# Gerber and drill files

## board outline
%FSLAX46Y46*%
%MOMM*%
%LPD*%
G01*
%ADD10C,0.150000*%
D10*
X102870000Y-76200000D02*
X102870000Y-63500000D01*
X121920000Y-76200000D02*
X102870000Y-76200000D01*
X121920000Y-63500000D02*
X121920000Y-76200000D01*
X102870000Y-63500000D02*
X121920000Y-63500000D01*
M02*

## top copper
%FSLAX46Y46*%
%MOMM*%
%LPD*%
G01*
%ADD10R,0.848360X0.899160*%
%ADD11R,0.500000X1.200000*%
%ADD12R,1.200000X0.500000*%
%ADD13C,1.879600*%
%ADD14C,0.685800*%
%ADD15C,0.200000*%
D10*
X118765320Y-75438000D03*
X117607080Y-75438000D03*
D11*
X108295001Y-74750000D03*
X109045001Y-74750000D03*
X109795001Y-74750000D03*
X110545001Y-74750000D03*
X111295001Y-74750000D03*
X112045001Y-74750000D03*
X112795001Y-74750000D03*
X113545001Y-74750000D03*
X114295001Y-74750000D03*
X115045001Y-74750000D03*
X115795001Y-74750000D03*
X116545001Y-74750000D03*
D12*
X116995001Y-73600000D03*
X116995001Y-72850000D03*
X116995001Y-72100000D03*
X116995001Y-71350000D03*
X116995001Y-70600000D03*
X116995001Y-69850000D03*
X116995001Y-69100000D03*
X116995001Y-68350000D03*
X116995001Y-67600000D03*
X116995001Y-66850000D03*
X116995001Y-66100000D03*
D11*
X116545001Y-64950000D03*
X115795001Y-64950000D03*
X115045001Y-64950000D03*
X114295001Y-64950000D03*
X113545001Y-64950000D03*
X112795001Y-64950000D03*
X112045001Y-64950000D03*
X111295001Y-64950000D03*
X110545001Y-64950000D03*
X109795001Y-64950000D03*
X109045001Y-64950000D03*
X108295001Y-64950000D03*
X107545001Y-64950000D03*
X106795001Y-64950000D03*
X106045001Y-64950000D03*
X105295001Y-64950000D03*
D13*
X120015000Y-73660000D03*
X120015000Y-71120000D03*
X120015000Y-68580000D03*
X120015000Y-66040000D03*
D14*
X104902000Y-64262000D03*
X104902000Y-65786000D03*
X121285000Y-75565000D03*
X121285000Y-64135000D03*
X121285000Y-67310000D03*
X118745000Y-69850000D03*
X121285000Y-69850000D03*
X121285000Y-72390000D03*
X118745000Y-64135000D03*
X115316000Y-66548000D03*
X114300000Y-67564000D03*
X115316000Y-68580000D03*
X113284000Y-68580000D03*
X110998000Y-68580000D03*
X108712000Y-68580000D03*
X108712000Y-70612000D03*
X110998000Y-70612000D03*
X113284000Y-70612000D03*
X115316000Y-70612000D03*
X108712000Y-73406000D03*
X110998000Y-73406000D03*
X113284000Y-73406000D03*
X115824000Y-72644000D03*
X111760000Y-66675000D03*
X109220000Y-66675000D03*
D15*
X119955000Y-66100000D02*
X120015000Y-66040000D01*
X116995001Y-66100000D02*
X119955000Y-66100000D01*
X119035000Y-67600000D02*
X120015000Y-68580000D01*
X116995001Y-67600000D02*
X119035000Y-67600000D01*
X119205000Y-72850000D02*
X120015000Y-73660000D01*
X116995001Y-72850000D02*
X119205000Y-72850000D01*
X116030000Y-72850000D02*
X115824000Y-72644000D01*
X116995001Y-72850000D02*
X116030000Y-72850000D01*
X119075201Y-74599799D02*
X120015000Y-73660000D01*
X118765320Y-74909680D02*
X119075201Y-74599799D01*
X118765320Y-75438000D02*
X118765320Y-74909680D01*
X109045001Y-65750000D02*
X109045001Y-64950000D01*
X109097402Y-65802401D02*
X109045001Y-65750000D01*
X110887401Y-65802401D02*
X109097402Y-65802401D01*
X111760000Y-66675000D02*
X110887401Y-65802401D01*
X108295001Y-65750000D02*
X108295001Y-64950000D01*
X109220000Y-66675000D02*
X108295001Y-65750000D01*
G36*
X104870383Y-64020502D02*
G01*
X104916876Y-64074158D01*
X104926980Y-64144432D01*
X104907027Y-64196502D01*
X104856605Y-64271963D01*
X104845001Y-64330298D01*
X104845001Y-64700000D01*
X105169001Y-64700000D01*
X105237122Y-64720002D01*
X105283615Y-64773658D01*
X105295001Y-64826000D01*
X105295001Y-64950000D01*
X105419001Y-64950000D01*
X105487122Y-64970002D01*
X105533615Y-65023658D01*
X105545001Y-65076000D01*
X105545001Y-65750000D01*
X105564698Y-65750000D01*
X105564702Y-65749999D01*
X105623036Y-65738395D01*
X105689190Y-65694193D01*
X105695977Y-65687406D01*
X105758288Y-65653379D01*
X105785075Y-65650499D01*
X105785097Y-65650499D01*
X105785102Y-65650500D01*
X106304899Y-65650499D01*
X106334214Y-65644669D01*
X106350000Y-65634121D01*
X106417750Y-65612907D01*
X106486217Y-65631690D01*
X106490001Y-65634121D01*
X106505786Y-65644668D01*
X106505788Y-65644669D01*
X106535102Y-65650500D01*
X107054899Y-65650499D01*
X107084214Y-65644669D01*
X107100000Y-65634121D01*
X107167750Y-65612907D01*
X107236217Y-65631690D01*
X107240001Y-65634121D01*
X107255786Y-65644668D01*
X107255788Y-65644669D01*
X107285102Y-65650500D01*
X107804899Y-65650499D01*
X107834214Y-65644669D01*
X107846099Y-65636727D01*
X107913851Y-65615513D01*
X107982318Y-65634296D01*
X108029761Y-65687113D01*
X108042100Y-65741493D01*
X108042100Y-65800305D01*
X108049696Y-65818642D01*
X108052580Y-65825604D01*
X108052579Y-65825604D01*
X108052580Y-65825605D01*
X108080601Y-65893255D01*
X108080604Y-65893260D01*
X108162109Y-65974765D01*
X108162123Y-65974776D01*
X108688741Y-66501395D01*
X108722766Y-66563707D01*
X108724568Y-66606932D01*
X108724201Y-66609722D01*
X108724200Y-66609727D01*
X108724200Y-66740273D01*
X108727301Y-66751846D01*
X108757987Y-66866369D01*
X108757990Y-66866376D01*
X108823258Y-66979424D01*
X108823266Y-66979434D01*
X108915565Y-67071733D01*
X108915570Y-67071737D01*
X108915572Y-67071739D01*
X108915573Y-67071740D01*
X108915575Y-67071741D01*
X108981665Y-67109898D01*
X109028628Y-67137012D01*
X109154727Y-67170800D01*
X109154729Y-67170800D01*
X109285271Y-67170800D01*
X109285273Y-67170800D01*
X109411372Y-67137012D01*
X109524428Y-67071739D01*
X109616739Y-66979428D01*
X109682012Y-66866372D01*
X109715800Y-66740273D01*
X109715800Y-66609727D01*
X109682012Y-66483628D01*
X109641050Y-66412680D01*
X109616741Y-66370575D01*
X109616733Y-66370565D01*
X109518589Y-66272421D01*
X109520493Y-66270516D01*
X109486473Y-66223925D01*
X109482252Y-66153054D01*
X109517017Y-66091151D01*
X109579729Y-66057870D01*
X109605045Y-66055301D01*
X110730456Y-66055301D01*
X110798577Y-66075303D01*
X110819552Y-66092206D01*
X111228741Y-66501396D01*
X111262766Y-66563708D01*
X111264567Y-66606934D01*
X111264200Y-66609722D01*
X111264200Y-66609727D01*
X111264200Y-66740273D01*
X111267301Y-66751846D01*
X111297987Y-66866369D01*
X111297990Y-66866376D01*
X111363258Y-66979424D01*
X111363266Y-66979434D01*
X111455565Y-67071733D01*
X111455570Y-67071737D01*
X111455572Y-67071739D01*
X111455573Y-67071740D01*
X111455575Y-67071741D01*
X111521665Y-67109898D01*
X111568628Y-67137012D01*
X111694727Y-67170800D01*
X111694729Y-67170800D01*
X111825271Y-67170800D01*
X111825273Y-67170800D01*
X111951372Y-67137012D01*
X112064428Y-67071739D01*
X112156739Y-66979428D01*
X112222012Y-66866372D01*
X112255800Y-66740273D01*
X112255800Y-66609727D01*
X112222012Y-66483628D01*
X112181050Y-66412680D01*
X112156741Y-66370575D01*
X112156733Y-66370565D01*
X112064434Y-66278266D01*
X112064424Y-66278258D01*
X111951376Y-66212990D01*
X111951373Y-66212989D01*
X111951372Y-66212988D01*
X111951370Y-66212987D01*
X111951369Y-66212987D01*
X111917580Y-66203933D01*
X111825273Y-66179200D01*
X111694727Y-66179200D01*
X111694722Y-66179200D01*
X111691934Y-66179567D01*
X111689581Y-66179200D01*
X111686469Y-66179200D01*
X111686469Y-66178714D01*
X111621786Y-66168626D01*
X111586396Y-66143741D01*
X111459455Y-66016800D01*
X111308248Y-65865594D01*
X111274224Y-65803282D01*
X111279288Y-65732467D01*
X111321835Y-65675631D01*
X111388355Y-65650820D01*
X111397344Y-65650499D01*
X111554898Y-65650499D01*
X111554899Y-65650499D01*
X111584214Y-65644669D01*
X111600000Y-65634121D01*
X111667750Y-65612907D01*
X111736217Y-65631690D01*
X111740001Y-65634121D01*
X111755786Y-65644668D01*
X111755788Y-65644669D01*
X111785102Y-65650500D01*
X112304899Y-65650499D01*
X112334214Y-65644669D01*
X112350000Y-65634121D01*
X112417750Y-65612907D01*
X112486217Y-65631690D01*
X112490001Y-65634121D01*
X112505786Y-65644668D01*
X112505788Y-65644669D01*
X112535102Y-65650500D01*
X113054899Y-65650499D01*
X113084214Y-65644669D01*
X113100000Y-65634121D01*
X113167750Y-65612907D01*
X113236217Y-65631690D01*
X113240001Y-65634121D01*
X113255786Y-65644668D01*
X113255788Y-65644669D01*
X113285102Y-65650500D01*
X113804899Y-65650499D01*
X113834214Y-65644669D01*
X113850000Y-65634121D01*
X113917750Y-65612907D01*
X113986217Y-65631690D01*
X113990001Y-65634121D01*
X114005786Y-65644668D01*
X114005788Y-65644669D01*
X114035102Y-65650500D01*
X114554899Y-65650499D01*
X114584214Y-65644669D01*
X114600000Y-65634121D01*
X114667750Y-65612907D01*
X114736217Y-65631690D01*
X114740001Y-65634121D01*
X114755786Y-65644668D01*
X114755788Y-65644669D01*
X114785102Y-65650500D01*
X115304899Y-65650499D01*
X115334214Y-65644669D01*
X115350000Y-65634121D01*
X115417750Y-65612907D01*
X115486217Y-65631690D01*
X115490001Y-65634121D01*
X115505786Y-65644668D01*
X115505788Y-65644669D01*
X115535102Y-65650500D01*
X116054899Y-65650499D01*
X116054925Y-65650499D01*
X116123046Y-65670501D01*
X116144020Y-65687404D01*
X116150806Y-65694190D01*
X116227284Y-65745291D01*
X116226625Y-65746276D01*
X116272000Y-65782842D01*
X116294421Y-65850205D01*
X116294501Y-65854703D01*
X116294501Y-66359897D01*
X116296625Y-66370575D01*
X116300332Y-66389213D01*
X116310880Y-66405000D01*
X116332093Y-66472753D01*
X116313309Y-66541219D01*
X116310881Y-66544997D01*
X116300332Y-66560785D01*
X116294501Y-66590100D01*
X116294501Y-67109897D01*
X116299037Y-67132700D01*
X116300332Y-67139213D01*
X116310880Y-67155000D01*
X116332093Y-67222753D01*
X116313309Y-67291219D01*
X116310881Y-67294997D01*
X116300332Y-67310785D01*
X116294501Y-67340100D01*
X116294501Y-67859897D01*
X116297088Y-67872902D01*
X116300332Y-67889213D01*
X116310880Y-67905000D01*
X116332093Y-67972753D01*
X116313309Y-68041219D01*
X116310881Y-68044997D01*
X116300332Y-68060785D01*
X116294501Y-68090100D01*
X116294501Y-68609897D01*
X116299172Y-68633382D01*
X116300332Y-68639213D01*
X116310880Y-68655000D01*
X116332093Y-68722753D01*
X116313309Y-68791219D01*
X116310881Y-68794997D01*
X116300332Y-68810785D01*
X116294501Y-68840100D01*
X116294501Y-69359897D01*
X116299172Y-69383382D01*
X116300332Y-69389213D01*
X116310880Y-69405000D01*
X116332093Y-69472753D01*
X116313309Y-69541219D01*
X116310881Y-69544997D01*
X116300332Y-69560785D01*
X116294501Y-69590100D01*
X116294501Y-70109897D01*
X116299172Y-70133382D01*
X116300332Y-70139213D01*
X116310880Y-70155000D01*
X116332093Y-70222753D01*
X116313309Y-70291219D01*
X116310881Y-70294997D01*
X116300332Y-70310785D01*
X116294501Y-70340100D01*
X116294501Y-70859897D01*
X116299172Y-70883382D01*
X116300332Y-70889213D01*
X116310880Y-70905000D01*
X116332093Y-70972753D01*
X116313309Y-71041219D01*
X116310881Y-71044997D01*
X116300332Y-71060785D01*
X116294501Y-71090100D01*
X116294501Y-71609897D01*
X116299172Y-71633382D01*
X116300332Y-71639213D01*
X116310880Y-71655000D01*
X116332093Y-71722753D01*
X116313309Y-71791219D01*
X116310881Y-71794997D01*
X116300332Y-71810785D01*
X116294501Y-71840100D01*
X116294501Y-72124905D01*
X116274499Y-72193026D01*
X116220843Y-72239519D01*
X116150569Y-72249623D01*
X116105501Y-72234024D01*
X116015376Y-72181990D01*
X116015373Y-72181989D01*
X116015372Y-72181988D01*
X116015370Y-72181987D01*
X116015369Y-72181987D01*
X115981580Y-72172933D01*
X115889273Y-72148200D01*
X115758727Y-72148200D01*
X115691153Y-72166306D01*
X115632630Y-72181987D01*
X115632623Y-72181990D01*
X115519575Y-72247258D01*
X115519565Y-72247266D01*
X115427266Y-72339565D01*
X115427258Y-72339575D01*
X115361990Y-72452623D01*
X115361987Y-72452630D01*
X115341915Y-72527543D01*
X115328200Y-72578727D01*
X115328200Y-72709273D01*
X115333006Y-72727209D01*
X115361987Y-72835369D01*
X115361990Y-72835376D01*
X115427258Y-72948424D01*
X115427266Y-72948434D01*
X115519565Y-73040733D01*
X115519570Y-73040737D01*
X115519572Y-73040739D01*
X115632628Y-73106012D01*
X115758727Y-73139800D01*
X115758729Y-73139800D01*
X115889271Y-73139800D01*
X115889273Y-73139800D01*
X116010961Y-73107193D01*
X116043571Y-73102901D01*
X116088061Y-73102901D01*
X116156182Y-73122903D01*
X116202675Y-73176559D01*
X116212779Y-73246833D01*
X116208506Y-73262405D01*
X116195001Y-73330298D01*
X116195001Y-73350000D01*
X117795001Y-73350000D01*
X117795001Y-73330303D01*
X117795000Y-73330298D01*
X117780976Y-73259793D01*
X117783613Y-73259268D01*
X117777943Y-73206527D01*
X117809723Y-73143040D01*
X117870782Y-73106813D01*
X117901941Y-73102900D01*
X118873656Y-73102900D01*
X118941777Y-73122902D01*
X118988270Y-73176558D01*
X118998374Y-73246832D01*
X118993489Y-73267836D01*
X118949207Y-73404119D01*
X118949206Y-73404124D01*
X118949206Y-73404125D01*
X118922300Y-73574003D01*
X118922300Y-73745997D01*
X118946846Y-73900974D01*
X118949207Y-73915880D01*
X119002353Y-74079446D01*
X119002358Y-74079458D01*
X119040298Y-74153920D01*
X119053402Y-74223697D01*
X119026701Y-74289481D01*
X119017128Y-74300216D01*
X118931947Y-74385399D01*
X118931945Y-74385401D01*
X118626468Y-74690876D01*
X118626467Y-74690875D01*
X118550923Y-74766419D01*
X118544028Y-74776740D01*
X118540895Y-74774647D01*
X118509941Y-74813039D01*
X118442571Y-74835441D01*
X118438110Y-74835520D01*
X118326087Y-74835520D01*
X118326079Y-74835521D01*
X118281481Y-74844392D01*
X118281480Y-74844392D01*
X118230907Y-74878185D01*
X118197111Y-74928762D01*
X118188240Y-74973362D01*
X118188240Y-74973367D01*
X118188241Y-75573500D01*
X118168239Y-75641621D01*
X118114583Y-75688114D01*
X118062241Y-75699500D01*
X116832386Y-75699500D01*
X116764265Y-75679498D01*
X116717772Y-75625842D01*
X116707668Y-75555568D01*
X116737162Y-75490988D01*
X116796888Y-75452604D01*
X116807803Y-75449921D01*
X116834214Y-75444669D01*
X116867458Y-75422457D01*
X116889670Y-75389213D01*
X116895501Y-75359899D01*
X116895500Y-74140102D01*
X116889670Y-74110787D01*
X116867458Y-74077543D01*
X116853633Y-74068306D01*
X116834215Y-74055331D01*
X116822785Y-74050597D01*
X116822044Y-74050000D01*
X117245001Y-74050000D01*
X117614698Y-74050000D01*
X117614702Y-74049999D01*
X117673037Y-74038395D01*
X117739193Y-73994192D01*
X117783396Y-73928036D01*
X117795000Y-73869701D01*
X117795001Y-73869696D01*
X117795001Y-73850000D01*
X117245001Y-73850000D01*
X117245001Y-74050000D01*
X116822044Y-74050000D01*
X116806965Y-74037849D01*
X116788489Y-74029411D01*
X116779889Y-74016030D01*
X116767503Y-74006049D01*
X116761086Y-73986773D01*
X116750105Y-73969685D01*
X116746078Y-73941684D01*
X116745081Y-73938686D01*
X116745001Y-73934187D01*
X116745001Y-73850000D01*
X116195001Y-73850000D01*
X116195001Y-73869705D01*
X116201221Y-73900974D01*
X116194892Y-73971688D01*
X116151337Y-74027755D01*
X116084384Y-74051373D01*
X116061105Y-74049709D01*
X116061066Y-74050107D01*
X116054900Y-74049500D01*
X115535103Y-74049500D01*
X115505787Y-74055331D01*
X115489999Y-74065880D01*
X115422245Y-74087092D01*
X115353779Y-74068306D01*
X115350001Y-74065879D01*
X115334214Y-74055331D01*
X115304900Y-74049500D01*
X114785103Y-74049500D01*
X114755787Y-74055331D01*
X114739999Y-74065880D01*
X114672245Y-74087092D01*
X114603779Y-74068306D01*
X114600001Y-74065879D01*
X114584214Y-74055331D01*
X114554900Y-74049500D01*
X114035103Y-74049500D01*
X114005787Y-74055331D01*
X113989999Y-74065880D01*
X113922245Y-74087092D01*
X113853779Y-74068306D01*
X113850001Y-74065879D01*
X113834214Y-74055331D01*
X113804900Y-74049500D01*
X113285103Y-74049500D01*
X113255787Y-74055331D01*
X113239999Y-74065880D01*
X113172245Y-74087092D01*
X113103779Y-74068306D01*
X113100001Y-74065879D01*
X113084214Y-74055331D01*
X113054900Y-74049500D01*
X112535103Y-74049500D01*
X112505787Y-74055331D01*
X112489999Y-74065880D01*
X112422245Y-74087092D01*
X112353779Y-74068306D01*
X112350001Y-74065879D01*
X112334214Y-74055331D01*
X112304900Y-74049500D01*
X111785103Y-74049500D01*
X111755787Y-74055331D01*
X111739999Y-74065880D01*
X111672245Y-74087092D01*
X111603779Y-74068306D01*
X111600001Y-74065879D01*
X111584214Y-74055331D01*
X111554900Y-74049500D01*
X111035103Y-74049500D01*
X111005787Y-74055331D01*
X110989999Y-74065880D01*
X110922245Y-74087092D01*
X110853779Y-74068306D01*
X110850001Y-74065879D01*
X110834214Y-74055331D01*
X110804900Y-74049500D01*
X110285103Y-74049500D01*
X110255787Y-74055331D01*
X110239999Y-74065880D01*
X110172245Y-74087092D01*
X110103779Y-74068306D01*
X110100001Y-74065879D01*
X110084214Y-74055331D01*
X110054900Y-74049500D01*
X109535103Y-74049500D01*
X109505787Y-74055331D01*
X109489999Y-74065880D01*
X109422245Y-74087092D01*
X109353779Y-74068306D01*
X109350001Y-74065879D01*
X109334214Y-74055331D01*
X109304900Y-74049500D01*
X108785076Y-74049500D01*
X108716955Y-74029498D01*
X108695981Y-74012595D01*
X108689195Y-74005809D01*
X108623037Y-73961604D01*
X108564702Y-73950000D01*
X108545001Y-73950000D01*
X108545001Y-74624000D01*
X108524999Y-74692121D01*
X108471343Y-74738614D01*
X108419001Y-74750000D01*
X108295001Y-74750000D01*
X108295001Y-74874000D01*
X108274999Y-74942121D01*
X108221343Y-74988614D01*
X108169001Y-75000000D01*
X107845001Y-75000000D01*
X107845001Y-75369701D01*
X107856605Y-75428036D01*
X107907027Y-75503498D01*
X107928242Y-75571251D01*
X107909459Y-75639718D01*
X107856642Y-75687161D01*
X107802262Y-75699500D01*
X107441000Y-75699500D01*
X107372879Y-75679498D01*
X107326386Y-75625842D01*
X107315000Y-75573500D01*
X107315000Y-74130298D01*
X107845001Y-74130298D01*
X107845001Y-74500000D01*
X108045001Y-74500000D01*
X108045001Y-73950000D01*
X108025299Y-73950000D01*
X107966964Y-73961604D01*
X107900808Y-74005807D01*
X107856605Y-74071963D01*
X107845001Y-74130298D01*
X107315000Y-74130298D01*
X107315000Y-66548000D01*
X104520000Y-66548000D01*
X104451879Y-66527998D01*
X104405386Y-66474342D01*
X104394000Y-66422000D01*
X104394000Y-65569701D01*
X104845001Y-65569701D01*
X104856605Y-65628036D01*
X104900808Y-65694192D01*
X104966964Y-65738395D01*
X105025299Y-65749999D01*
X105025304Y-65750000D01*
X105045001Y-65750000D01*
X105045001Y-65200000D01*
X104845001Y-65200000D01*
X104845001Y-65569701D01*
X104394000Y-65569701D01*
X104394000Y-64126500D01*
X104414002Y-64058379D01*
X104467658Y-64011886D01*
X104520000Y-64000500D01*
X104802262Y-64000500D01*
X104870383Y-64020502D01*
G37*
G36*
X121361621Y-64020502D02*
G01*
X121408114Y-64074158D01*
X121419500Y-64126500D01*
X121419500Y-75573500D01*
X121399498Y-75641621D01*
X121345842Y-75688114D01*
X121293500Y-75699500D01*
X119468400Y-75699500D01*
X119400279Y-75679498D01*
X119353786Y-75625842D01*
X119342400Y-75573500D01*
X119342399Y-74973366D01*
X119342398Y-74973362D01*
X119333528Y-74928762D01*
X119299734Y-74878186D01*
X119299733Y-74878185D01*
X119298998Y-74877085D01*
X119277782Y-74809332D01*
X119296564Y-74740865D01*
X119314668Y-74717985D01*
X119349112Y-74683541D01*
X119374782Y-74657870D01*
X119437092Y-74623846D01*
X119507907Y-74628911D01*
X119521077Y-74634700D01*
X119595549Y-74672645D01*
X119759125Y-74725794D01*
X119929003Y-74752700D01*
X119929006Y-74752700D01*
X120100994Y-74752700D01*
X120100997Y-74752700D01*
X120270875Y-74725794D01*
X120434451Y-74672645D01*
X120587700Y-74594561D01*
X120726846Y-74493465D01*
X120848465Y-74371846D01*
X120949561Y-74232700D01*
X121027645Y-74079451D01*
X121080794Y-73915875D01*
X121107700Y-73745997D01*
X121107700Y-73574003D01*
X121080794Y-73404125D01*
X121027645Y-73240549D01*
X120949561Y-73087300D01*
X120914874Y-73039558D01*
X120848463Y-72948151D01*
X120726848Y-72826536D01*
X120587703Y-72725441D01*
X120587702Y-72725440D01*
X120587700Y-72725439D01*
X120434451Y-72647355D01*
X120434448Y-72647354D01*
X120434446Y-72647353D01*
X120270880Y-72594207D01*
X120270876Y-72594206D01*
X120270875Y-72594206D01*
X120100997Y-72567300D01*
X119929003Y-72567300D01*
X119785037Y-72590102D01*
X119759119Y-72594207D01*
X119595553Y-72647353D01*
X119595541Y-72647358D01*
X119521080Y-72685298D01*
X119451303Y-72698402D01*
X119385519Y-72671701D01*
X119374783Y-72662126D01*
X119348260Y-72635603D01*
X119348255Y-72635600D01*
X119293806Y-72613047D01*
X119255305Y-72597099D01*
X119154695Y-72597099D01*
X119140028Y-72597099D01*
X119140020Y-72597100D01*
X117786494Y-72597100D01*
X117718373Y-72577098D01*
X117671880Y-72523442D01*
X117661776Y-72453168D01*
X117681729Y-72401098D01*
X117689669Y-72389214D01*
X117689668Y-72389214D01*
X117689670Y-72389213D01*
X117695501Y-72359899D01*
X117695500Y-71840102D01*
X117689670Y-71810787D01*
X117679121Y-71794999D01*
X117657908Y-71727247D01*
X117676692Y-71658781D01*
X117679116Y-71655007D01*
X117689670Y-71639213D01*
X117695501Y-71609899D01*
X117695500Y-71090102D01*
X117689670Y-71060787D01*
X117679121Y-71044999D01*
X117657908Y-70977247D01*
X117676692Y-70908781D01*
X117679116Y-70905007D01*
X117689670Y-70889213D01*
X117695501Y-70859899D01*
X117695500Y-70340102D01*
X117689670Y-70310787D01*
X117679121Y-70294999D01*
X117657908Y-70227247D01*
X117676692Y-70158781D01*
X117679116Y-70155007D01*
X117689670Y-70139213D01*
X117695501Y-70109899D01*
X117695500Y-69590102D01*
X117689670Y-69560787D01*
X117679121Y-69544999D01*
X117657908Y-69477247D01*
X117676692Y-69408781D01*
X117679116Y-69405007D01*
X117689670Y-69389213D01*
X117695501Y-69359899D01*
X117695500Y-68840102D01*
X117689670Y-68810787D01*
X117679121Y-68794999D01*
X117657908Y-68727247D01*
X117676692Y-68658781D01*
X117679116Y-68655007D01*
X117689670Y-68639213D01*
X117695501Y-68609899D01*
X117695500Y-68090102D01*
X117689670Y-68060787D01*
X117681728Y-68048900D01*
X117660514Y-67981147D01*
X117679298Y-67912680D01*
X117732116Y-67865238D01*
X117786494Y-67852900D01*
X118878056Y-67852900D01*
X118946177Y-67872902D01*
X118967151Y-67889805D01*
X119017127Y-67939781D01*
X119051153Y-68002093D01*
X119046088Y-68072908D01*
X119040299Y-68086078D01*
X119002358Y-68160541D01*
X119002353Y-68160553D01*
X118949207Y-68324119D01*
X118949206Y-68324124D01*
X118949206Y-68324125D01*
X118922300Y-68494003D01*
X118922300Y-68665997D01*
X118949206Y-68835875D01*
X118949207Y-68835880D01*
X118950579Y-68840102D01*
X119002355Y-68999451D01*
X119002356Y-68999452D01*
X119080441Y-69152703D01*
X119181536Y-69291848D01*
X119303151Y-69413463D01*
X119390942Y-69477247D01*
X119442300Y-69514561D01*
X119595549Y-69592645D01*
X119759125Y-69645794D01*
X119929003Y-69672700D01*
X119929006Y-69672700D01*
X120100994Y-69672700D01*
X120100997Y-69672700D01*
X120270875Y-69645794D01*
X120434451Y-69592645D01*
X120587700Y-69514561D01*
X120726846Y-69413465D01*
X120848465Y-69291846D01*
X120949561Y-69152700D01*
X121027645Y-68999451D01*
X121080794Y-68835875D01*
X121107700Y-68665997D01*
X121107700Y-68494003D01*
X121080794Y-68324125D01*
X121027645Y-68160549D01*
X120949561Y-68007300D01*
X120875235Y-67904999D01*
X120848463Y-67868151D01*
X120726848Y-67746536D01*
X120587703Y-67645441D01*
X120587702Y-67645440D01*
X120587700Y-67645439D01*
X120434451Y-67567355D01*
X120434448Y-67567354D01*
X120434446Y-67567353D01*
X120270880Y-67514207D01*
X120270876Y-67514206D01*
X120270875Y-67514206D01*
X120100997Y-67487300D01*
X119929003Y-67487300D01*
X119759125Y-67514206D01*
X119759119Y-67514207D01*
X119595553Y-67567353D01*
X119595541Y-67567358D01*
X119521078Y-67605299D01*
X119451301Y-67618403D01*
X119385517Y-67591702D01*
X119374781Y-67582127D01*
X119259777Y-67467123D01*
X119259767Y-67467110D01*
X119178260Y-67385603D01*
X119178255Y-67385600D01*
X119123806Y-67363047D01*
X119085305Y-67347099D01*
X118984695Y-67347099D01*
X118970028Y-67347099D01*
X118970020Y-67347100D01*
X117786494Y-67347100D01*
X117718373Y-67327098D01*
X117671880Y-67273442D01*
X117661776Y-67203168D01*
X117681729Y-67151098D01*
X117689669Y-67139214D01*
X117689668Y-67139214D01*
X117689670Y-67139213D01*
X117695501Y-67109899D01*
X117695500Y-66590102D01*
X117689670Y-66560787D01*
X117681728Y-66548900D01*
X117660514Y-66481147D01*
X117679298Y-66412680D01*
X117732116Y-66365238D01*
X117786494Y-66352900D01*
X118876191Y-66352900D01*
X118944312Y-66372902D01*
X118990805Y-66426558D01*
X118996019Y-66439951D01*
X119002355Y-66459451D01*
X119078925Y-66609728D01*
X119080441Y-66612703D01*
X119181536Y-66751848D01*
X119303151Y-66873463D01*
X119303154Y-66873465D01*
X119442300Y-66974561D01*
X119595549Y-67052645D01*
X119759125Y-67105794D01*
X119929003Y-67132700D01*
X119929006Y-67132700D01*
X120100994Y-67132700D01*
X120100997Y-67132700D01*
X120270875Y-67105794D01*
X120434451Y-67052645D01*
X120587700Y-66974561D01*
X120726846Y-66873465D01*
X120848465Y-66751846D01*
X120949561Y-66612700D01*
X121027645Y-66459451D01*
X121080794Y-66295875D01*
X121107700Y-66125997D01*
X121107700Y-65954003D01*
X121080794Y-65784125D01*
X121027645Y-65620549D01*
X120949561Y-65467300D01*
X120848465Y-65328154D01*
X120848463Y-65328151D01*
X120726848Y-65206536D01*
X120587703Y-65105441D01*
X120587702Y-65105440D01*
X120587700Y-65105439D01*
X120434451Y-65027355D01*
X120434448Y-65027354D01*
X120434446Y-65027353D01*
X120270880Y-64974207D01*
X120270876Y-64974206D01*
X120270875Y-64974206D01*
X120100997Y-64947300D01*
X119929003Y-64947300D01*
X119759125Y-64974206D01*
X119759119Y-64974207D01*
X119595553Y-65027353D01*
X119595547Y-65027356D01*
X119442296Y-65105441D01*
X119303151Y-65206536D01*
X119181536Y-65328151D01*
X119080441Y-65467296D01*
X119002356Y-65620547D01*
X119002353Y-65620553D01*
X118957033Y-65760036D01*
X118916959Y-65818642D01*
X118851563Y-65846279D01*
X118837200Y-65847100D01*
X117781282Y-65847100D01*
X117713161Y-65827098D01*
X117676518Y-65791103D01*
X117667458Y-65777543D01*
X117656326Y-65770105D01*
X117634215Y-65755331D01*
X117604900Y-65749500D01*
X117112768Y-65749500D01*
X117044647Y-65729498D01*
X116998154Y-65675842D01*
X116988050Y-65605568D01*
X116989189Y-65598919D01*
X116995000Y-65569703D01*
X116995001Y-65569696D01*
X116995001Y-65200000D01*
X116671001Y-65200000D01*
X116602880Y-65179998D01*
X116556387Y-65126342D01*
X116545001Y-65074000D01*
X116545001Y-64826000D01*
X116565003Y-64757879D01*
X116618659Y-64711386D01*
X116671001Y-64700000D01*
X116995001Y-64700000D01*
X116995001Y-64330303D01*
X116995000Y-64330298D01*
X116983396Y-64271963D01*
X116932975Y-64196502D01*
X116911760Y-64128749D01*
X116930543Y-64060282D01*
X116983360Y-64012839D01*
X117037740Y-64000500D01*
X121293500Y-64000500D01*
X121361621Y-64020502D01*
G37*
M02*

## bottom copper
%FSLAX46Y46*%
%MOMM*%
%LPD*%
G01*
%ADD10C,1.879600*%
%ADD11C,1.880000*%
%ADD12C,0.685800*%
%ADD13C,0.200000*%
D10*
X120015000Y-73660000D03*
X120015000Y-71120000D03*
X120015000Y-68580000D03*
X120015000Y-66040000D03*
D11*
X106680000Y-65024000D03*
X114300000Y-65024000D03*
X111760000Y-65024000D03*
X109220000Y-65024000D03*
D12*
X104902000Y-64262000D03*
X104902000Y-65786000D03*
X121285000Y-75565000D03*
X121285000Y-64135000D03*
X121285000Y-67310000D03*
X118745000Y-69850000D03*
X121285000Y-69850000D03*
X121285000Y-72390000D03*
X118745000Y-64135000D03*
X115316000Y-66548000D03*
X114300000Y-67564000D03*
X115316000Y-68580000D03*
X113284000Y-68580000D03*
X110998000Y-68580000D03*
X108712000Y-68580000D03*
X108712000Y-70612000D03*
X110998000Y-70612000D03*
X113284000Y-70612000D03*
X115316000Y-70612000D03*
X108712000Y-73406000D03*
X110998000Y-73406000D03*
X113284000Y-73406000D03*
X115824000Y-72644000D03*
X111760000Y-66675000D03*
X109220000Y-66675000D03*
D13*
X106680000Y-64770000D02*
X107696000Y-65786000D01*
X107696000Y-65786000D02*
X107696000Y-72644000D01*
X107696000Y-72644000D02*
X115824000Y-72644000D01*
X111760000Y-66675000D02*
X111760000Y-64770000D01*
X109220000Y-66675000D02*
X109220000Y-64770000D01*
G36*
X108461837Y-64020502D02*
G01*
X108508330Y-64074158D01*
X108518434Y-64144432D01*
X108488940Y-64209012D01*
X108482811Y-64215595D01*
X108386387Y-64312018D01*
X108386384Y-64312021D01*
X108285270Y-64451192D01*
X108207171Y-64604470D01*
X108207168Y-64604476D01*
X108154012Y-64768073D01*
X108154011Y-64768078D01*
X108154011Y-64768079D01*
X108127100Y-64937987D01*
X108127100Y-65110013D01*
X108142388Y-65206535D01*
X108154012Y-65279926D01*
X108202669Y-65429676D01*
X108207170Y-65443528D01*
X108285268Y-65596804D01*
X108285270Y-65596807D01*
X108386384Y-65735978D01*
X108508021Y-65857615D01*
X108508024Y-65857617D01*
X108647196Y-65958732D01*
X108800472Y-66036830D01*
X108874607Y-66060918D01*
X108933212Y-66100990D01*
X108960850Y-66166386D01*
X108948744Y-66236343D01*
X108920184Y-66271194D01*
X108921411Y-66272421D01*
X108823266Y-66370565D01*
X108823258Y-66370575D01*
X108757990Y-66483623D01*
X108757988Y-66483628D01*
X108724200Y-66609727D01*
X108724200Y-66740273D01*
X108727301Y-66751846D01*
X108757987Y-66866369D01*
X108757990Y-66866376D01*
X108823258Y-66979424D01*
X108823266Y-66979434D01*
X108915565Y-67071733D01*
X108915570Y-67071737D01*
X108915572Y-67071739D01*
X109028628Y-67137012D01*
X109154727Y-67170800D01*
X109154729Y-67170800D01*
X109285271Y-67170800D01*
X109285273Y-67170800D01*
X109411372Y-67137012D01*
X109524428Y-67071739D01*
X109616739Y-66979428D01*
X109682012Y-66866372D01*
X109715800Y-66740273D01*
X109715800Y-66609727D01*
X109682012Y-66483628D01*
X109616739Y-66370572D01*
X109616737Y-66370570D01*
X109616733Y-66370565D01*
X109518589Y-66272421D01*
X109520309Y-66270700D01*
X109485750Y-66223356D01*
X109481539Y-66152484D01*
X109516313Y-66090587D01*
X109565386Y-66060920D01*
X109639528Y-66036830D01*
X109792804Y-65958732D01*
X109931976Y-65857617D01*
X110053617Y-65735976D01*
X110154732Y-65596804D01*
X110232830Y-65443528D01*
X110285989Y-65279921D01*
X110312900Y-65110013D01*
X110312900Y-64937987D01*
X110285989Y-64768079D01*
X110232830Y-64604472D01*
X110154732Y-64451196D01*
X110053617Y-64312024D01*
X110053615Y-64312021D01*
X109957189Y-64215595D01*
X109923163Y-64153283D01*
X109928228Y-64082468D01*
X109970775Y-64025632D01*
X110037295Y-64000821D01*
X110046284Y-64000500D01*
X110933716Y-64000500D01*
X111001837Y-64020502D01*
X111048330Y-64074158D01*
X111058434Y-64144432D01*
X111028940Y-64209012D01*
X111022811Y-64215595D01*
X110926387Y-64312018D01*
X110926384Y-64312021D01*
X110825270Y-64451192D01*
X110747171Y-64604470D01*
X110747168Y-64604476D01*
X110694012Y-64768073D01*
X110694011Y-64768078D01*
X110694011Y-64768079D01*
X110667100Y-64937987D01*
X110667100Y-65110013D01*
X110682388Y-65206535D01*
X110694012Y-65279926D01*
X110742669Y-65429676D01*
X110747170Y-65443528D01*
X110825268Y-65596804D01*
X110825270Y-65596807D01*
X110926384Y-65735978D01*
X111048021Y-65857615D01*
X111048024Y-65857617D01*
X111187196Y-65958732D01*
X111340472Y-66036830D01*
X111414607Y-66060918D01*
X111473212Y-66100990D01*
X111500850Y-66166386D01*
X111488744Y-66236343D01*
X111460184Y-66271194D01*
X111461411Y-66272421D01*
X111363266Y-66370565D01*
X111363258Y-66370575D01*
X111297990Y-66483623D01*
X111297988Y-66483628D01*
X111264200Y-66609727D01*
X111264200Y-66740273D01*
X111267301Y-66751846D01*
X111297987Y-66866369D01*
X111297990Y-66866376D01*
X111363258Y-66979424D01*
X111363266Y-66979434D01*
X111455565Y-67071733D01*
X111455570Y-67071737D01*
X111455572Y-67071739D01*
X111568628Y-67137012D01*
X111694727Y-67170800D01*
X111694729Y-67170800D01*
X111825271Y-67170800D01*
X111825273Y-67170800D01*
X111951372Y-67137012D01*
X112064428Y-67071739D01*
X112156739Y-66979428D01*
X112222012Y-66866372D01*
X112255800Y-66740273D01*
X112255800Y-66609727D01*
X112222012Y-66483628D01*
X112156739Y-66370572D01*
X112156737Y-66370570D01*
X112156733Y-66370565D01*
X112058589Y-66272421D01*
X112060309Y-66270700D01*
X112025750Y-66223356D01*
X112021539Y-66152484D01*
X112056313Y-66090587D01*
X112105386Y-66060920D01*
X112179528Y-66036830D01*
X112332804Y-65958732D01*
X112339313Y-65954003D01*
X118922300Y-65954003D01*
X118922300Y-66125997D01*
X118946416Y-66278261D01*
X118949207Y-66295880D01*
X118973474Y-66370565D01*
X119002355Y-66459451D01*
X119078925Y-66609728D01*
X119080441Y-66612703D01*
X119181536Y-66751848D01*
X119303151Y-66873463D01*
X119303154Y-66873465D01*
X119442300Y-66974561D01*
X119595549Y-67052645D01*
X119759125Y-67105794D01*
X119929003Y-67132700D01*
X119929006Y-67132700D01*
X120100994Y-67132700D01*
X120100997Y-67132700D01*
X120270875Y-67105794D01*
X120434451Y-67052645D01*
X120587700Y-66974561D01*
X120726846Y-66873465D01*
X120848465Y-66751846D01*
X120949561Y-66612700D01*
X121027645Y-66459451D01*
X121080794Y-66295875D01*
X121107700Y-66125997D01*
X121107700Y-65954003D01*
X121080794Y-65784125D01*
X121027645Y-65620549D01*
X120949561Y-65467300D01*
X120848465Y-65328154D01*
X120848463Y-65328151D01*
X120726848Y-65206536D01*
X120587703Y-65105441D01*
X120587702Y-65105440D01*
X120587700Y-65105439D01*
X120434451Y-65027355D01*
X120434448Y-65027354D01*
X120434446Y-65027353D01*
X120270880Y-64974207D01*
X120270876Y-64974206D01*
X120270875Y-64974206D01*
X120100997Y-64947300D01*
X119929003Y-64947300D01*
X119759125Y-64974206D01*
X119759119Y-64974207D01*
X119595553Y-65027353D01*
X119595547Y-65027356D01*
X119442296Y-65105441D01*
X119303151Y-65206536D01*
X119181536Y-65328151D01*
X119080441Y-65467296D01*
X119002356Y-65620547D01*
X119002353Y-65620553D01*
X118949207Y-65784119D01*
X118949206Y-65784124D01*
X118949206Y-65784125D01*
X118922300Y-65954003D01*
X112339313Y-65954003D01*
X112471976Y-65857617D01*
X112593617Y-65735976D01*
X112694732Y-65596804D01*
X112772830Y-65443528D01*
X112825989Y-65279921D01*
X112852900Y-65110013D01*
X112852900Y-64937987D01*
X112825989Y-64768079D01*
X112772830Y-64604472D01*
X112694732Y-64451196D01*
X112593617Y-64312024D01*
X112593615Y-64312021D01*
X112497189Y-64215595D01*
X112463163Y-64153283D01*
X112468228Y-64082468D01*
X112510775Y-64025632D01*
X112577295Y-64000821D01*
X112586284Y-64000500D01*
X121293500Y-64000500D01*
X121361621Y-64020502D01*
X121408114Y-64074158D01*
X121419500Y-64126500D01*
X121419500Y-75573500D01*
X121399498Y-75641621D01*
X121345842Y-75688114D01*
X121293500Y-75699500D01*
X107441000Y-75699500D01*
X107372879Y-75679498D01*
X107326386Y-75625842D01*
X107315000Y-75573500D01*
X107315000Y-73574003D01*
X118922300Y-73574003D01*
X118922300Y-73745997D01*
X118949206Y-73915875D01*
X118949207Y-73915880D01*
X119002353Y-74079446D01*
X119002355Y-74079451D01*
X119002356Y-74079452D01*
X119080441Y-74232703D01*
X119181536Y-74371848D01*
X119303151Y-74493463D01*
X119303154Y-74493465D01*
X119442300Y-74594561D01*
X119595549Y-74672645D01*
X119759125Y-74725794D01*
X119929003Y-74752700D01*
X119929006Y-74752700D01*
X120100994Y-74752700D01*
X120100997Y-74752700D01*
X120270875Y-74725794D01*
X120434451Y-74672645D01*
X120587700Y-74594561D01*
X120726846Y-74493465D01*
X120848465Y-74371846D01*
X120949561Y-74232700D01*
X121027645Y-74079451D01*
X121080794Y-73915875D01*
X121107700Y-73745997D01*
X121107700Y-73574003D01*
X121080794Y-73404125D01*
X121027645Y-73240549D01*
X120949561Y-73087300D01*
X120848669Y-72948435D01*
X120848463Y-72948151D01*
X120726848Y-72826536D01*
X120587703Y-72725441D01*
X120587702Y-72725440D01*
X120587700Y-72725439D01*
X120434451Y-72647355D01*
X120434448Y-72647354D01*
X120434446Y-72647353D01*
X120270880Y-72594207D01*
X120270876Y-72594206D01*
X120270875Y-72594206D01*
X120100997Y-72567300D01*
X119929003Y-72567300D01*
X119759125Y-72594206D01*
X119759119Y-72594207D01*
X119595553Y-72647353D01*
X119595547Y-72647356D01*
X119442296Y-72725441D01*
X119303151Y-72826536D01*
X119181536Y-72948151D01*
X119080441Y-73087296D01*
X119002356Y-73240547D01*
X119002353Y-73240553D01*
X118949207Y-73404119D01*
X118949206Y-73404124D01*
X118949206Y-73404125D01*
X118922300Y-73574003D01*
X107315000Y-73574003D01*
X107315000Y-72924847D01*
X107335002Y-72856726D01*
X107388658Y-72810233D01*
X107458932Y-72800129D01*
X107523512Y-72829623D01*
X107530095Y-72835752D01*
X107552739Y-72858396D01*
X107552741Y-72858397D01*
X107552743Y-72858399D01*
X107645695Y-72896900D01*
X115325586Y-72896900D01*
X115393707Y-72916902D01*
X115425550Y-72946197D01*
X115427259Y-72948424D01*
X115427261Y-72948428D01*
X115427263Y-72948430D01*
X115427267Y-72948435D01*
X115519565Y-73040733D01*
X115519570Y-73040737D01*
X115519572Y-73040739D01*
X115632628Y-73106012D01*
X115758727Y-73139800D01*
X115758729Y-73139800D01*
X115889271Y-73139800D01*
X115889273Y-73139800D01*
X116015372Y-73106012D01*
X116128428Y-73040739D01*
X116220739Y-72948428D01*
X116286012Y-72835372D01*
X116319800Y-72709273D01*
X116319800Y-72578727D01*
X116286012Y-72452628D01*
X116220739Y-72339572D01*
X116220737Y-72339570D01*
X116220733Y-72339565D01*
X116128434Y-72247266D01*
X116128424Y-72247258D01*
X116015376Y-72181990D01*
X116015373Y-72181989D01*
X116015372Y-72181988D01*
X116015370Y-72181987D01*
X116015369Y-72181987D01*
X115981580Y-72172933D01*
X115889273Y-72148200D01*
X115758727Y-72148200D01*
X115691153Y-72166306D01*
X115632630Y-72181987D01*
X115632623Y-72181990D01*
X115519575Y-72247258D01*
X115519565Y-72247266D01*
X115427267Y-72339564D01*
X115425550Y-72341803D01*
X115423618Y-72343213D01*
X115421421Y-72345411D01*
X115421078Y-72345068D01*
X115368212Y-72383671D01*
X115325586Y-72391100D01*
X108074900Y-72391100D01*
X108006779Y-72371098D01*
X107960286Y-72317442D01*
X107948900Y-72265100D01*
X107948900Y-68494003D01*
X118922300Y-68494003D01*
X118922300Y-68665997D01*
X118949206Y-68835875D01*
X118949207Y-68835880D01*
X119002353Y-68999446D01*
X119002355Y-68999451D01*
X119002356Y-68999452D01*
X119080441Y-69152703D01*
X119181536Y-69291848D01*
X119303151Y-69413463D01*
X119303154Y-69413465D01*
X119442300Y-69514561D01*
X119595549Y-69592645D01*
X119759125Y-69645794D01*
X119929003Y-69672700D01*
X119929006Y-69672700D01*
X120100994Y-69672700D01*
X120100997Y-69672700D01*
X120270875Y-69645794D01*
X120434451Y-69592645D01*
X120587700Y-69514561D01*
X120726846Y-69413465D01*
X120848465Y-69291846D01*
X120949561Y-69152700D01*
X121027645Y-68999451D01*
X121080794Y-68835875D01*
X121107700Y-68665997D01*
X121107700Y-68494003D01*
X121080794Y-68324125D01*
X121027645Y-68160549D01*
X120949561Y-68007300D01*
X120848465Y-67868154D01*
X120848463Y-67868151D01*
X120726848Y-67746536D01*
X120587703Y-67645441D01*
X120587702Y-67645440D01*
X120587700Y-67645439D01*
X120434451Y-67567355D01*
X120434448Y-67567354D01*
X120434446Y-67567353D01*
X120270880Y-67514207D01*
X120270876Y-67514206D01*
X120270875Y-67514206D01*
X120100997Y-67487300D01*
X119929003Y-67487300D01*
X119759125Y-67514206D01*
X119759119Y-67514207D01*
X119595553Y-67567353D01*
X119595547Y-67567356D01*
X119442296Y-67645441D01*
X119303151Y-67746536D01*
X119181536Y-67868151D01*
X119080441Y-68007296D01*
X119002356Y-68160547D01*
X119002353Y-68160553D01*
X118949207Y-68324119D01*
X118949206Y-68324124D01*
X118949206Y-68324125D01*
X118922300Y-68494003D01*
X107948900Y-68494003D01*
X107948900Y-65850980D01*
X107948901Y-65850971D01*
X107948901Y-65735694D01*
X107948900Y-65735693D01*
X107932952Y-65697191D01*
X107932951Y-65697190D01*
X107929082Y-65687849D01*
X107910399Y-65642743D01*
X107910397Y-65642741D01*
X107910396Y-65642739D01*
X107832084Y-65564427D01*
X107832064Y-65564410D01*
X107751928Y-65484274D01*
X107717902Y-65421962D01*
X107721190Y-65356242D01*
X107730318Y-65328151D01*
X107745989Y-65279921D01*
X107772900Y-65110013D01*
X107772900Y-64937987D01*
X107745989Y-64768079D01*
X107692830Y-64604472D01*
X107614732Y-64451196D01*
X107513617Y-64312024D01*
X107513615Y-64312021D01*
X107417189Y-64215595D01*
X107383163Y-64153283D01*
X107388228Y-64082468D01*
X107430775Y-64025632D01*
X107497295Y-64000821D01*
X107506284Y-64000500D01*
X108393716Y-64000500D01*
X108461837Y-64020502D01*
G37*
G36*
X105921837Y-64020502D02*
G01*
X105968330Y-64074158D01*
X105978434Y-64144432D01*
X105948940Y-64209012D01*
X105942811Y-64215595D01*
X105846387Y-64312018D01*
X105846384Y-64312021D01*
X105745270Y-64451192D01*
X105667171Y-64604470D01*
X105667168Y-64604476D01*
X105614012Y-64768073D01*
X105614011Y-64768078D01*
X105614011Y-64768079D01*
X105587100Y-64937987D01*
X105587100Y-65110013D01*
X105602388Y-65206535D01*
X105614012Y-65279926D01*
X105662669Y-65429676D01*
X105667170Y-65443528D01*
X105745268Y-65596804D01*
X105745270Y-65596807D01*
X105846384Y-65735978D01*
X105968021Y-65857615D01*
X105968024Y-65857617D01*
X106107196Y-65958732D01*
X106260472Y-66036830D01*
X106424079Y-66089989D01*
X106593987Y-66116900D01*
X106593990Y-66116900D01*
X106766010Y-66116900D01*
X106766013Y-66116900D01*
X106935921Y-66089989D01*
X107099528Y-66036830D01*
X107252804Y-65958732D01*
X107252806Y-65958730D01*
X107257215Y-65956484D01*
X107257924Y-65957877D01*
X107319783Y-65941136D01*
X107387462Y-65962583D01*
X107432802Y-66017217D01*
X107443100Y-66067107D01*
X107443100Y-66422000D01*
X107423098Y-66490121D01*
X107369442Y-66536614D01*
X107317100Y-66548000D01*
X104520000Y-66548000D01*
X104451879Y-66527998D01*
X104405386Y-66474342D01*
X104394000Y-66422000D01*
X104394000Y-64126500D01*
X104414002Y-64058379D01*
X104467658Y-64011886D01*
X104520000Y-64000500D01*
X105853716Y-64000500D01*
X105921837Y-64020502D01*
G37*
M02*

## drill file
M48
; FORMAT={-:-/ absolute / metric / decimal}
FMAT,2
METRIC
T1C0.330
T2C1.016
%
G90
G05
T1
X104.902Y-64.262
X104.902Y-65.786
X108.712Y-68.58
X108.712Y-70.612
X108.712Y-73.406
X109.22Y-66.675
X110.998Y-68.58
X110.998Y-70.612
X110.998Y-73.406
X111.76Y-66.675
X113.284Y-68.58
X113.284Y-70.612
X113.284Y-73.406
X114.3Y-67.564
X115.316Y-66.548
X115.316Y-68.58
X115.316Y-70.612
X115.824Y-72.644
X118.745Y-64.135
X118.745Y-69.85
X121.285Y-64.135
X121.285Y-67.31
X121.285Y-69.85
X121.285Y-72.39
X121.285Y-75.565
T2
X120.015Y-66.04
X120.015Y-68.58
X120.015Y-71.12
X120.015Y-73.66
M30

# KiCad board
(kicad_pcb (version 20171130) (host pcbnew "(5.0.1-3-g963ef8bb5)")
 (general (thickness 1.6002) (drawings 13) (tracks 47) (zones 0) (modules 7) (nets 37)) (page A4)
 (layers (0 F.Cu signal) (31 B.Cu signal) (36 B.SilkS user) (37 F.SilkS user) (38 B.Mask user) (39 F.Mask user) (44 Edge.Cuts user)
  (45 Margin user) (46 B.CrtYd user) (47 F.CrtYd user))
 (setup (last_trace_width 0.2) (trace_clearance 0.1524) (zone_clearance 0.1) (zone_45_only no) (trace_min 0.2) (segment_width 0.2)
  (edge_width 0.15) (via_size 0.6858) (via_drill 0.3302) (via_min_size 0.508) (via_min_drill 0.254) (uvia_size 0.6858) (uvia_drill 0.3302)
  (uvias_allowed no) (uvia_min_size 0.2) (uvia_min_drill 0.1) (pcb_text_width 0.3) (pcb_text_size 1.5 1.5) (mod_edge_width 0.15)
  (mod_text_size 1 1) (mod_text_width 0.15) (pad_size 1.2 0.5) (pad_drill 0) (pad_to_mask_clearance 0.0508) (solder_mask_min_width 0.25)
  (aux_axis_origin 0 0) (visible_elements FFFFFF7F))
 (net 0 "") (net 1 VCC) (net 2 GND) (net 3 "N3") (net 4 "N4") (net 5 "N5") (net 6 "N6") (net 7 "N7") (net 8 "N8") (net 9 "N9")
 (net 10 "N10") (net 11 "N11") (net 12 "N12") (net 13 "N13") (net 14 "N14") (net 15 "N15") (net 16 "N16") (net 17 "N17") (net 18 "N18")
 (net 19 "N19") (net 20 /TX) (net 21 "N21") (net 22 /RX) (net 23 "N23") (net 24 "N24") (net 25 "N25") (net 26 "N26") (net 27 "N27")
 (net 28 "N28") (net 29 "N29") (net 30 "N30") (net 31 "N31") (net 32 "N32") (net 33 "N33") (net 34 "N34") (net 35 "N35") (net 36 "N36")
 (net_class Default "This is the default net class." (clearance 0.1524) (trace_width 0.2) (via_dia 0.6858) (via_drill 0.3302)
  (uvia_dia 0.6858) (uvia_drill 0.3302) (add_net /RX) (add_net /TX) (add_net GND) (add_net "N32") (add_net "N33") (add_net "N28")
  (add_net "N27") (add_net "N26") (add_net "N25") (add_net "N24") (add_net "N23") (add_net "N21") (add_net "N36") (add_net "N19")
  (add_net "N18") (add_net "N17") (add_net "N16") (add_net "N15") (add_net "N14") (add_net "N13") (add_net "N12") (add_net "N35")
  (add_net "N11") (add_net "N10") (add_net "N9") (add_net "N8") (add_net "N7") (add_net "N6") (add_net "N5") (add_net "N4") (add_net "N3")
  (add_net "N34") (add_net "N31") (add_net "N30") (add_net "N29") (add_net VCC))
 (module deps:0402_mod (layer F.Cu) (at 118.1862 75.438 180)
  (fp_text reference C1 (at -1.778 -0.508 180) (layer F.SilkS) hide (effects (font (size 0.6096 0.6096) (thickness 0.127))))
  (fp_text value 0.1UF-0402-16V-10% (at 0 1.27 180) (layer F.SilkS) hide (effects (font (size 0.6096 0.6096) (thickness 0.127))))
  (pad 1 smd rect (at -0.57912 0 180) (size 0.84836 0.89916) (layers F.Cu F.Paste F.Mask) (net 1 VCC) (solder_mask_margin 0.1016))
  (pad 2 smd rect (at 0.57912 0 180) (size 0.84836 0.89916) (layers F.Cu F.Paste F.Mask) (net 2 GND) (solder_mask_margin 0.1016)))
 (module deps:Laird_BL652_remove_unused (layer F.Cu) (at 111.145001 69.85) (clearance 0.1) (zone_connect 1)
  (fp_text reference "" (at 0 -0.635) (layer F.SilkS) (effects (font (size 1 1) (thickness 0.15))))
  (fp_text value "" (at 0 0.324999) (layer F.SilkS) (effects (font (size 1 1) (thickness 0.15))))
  (pad 39 smd rect (at -2.85 4.9 90) (size 1.2 0.5) (layers F.Cu F.Paste F.Mask) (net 2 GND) (zone_connect 1))
  (pad 38 smd rect (at -2.1 4.9 90) (size 1.2 0.5) (layers F.Cu F.Paste F.Mask) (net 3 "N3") (zone_connect 1))
  (pad 37 smd rect (at -1.35 4.9 90) (size 1.2 0.5) (layers F.Cu F.Paste F.Mask) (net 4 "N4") (zone_connect 1))
  (pad 36 smd rect (at -0.6 4.9 90) (size 1.2 0.5) (layers F.Cu F.Paste F.Mask) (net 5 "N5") (zone_connect 1))
  (pad 35 smd rect (at 0.15 4.9 90) (size 1.2 0.5) (layers F.Cu F.Paste F.Mask) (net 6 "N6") (zone_connect 1))
  (pad 34 smd rect (at 0.9 4.9 90) (size 1.2 0.5) (layers F.Cu F.Paste F.Mask) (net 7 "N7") (zone_connect 1))
  (pad 33 smd rect (at 1.65 4.9 90) (size 1.2 0.5) (layers F.Cu F.Paste F.Mask) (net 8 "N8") (zone_connect 1))
  (pad 32 smd rect (at 2.4 4.9 90) (size 1.2 0.5) (layers F.Cu F.Paste F.Mask) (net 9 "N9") (zone_connect 1))
  (pad 31 smd rect (at 3.15 4.9 90) (size 1.2 0.5) (layers F.Cu F.Paste F.Mask) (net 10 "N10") (zone_connect 1))
  (pad 30 smd rect (at 3.9 4.9 90) (size 1.2 0.5) (layers F.Cu F.Paste F.Mask) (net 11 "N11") (zone_connect 1))
  (pad 29 smd rect (at 4.65 4.9 90) (size 1.2 0.5) (layers F.Cu F.Paste F.Mask) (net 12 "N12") (zone_connect 1))
  (pad 28 smd rect (at 5.4 4.9 90) (size 1.2 0.5) (layers F.Cu F.Paste F.Mask) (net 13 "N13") (zone_connect 1))
  (pad 27 smd rect (at 5.85 3.75) (size 1.2 0.5) (layers F.Cu F.Paste F.Mask) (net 2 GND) (zone_connect 1))
  (pad 26 smd rect (at 5.85 3) (size 1.2 0.5) (layers F.Cu F.Paste F.Mask) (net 1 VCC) (zone_connect 1))
  (pad 25 smd rect (at 5.85 2.25) (size 1.2 0.5) (layers F.Cu F.Paste F.Mask) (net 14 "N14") (zone_connect 1))
  (pad 24 smd rect (at 5.85 1.5) (size 1.2 0.5) (layers F.Cu F.Paste F.Mask) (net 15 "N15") (zone_connect 1))
  (pad 23 smd rect (at 5.85 0.75) (size 1.2 0.5) (layers F.Cu F.Paste F.Mask) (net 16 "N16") (zone_connect 1))
  (pad 22 smd rect (at 5.85 0) (size 1.2 0.5) (layers F.Cu F.Paste F.Mask) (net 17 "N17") (zone_connect 1))
  (pad 21 smd rect (at 5.85 -0.75) (size 1.2 0.5) (layers F.Cu F.Paste F.Mask) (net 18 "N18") (zone_connect 1))
  (pad 20 smd rect (at 5.85 -1.5) (size 1.2 0.5) (layers F.Cu F.Paste F.Mask) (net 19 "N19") (zone_connect 1))
  (pad 19 smd rect (at 5.85 -2.25) (size 1.2 0.5) (layers F.Cu F.Paste F.Mask) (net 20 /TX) (zone_connect 1))
  (pad 18 smd rect (at 5.85 -3) (size 1.2 0.5) (layers F.Cu F.Paste F.Mask) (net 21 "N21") (zone_connect 1))
  (pad 17 smd rect (at 5.85 -3.75) (size 1.2 0.5) (layers F.Cu F.Paste F.Mask) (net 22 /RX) (zone_connect 1))
  (pad 16 smd rect (at 5.4 -4.9 90) (size 1.2 0.5) (layers F.Cu F.Paste F.Mask) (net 2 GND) (zone_connect 1))
  (pad 15 smd rect (at 4.65 -4.9 90) (size 1.2 0.5) (layers F.Cu F.Paste F.Mask) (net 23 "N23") (zone_connect 1))
  (pad 14 smd rect (at 3.9 -4.9 90) (size 1.2 0.5) (layers F.Cu F.Paste F.Mask) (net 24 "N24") (zone_connect 1))
  (pad 13 smd rect (at 3.15 -4.9 90) (size 1.2 0.5) (layers F.Cu F.Paste F.Mask) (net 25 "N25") (zone_connect 1))
  (pad 12 smd rect (at 2.4 -4.9 90) (size 1.2 0.5) (layers F.Cu F.Paste F.Mask) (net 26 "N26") (zone_connect 1))
  (pad 11 smd rect (at 1.65 -4.9 90) (size 1.2 0.5) (layers F.Cu F.Paste F.Mask) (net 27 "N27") (zone_connect 1))
  (pad 10 smd rect (at 0.9 -4.9 90) (size 1.2 0.5) (layers F.Cu F.Paste F.Mask) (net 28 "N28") (zone_connect 1))
  (pad 9 smd rect (at 0.15 -4.9 90) (size 1.2 0.5) (layers F.Cu F.Paste F.Mask) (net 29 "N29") (zone_connect 1))
  (pad 8 smd rect (at -0.6 -4.9 90) (size 1.2 0.5) (layers F.Cu F.Paste F.Mask) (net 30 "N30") (zone_connect 1))
  (pad 7 smd rect (at -1.35 -4.9 90) (size 1.2 0.5) (layers F.Cu F.Paste F.Mask) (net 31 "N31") (zone_connect 1))
  (pad 6 smd rect (at -2.1 -4.9 90) (size 1.2 0.5) (layers F.Cu F.Paste F.Mask) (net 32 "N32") (zone_connect 1))
  (pad 5 smd rect (at -2.85 -4.9 90) (size 1.2 0.5) (layers F.Cu F.Paste F.Mask) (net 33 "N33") (zone_connect 1))
  (pad 4 smd rect (at -3.6 -4.9 90) (size 1.2 0.5) (layers F.Cu F.Paste F.Mask) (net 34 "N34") (zone_connect 1))
  (pad 3 smd rect (at -4.35 -4.9 90) (size 1.2 0.5) (layers F.Cu F.Paste F.Mask) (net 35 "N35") (zone_connect 1))
  (pad 2 smd rect (at -5.1 -4.9 90) (size 1.2 0.5) (layers F.Cu F.Paste F.Mask) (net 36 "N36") (zone_connect 1))
  (pad 1 smd rect (at -5.85 -4.9 90) (size 1.2 0.5) (layers F.Cu F.Paste F.Mask) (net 2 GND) (zone_connect 1)))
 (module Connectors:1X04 (layer F.Cu) (at 120.015 66.04 270)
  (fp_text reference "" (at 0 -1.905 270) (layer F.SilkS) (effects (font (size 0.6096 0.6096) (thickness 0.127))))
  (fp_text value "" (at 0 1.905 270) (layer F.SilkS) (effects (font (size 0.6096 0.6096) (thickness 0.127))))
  (pad 4 thru_hole circle (at 7.62 0 270) (size 1.8796 1.8796) (drill 1.016) (layers *.Cu *.Mask) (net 1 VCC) (solder_mask_margin 0.1016))
  (pad 3 thru_hole circle (at 5.08 0 270) (size 1.8796 1.8796) (drill 1.016) (layers *.Cu *.Mask) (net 2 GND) (solder_mask_margin 0.1016))
  (pad 2 thru_hole circle (at 2.54 0 270) (size 1.8796 1.8796) (drill 1.016) (layers *.Cu *.Mask) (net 20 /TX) (solder_mask_margin 0.1016))
  (pad 1 thru_hole circle (at 0 0 270) (size 1.8796 1.8796) (drill 1.016) (layers *.Cu *.Mask) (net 22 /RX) (solder_mask_margin 0.1016)))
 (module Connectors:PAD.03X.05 (layer B.Cu) (at 106.68 65.024)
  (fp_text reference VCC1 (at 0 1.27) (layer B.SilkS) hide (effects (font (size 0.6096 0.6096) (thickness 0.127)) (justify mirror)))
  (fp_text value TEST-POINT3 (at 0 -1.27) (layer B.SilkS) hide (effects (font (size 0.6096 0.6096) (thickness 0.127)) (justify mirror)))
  (pad P$1 smd circle (at 0 0) (size 1.88 1.88) (layers B.Cu B.Paste B.Mask) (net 1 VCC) (solder_mask_margin 0.1016)))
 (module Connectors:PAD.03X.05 (layer B.Cu) (at 114.3 65.024 180)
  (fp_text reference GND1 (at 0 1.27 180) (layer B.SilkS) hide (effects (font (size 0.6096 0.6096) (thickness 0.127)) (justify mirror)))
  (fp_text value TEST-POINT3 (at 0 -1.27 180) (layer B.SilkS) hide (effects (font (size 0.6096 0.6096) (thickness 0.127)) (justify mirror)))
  (pad P$1 smd circle (at 0 0 180) (size 1.88 1.88) (layers B.Cu B.Paste B.Mask) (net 2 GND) (solder_mask_margin 0.1016)))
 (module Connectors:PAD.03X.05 (layer B.Cu) (at 111.76 65.024)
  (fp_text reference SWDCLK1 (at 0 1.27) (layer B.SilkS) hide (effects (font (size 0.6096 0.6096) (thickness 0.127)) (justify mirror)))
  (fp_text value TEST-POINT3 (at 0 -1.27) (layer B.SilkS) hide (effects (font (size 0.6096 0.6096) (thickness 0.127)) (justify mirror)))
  (pad P$1 smd circle (at 0 0) (size 1.88 1.88) (layers B.Cu B.Paste B.Mask) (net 32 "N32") (solder_mask_margin 0.1016)))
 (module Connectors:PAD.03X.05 (layer B.Cu) (at 109.22 65.024 180)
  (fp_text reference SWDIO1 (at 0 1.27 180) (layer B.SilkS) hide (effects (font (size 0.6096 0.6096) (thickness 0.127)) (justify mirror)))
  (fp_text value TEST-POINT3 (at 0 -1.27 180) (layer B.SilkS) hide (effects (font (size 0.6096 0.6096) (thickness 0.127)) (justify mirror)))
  (pad P$1 smd circle (at 0 0 180) (size 1.88 1.88) (layers B.Cu B.Paste B.Mask) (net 33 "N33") (solder_mask_margin 0.1016)))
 (gr_line (start 102.87 76.2) (end 102.87 63.5) (layer Edge.Cuts) (width 0.15))
 (gr_line (start 121.92 76.2) (end 102.87 76.2) (layer Edge.Cuts) (width 0.15))
 (gr_line (start 121.92 63.5) (end 121.92 76.2) (layer Edge.Cuts) (width 0.15))
 (gr_line (start 102.87 63.5) (end 121.92 63.5) (layer Edge.Cuts) (width 0.15))
 (via (at 104.902 64.262) (size 0.6858) (drill 0.3302) (layers F.Cu B.Cu) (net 2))
 (via (at 104.902 65.786) (size 0.6858) (drill 0.3302) (layers F.Cu B.Cu) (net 2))
 (via (at 121.285 75.565) (size 0.6858) (drill 0.3302) (layers F.Cu B.Cu) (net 2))
 (via (at 121.285 64.135) (size 0.6858) (drill 0.3302) (layers F.Cu B.Cu) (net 2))
 (via (at 121.285 67.31) (size 0.6858) (drill 0.3302) (layers F.Cu B.Cu) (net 2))
 (via (at 118.745 69.85) (size 0.6858) (drill 0.3302) (layers F.Cu B.Cu) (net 2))
 (via (at 121.285 69.85) (size 0.6858) (drill 0.3302) (layers F.Cu B.Cu) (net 2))
 (via (at 121.285 72.39) (size 0.6858) (drill 0.3302) (layers F.Cu B.Cu) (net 2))
 (via (at 118.745 64.135) (size 0.6858) (drill 0.3302) (layers F.Cu B.Cu) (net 2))
 (via (at 115.316 66.548) (size 0.6858) (drill 0.3302) (layers F.Cu B.Cu) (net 2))
 (via (at 114.3 67.564) (size 0.6858) (drill 0.3302) (layers F.Cu B.Cu) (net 2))
 (via (at 115.316 68.58) (size 0.6858) (drill 0.3302) (layers F.Cu B.Cu) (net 2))
 (via (at 113.284 68.58) (size 0.6858) (drill 0.3302) (layers F.Cu B.Cu) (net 2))
 (via (at 110.998 68.58) (size 0.6858) (drill 0.3302) (layers F.Cu B.Cu) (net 2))
 (via (at 108.712 68.58) (size 0.6858) (drill 0.3302) (layers F.Cu B.Cu) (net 2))
 (via (at 108.712 70.612) (size 0.6858) (drill 0.3302) (layers F.Cu B.Cu) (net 2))
 (via (at 110.998 70.612) (size 0.6858) (drill 0.3302) (layers F.Cu B.Cu) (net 2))
 (via (at 113.284 70.612) (size 0.6858) (drill 0.3302) (layers F.Cu B.Cu) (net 2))
 (via (at 115.316 70.612) (size 0.6858) (drill 0.3302) (layers F.Cu B.Cu) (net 2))
 (via (at 108.712 73.406) (size 0.6858) (drill 0.3302) (layers F.Cu B.Cu) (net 2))
 (via (at 110.998 73.406) (size 0.6858) (drill 0.3302) (layers F.Cu B.Cu) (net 2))
 (via (at 113.284 73.406) (size 0.6858) (drill 0.3302) (layers F.Cu B.Cu) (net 2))
 (segment (start 119.955 66.1) (end 120.015 66.04) (width 0.2) (layer F.Cu) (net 22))
 (segment (start 116.995001 66.1) (end 119.955 66.1) (width 0.2) (layer F.Cu) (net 22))
 (segment (start 119.035 67.6) (end 120.015 68.58) (width 0.2) (layer F.Cu) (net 20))
 (segment (start 116.995001 67.6) (end 119.035 67.6) (width 0.2) (layer F.Cu) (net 20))
 (via (at 115.824 72.644) (size 0.6858) (drill 0.3302) (layers F.Cu B.Cu) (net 1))
 (segment (start 119.205 72.85) (end 120.015 73.66) (width 0.2) (layer F.Cu) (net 1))
 (segment (start 116.995001 72.85) (end 119.205 72.85) (width 0.2) (layer F.Cu) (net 1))
 (segment (start 116.03 72.85) (end 115.824 72.644) (width 0.2) (layer F.Cu) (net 1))
 (segment (start 116.995001 72.85) (end 116.03 72.85) (width 0.2) (layer F.Cu) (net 1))
 (segment (start 106.68 64.77) (end 107.696 65.786) (width 0.2) (layer B.Cu) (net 1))
 (segment (start 107.696 65.786) (end 107.696 72.644) (width 0.2) (layer B.Cu) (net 1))
 (segment (start 107.696 72.644) (end 115.824 72.644) (width 0.2) (layer B.Cu) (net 1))
 (segment (start 119.075201 74.599799) (end 120.015 73.66) (width 0.2) (layer F.Cu) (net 1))
 (segment (start 118.76532 74.90968) (end 119.075201 74.599799) (width 0.2) (layer F.Cu) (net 1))
 (segment (start 118.76532 75.438) (end 118.76532 74.90968) (width 0.2) (layer F.Cu) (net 1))
 (via (at 111.76 66.675) (size 0.6858) (drill 0.3302) (layers F.Cu B.Cu) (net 32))
 (segment (start 111.76 66.675) (end 111.76 64.77) (width 0.2) (layer B.Cu) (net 32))
 (segment (start 109.045001 65.75) (end 109.045001 64.95) (width 0.2) (layer F.Cu) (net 32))
 (segment (start 109.097402 65.802401) (end 109.045001 65.75) (width 0.2) (layer F.Cu) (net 32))
 (segment (start 110.887401 65.802401) (end 109.097402 65.802401) (width 0.2) (layer F.Cu) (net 32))
 (segment (start 111.76 66.675) (end 110.887401 65.802401) (width 0.2) (layer F.Cu) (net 32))
 (via (at 109.22 66.675) (size 0.6858) (drill 0.3302) (layers F.Cu B.Cu) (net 33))
 (segment (start 109.22 66.675) (end 109.22 64.77) (width 0.2) (layer B.Cu) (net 33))
 (segment (start 108.295001 65.75) (end 108.295001 64.95) (width 0.2) (layer F.Cu) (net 33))
 (segment (start 109.22 66.675) (end 108.295001 65.75) (width 0.2) (layer F.Cu) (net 33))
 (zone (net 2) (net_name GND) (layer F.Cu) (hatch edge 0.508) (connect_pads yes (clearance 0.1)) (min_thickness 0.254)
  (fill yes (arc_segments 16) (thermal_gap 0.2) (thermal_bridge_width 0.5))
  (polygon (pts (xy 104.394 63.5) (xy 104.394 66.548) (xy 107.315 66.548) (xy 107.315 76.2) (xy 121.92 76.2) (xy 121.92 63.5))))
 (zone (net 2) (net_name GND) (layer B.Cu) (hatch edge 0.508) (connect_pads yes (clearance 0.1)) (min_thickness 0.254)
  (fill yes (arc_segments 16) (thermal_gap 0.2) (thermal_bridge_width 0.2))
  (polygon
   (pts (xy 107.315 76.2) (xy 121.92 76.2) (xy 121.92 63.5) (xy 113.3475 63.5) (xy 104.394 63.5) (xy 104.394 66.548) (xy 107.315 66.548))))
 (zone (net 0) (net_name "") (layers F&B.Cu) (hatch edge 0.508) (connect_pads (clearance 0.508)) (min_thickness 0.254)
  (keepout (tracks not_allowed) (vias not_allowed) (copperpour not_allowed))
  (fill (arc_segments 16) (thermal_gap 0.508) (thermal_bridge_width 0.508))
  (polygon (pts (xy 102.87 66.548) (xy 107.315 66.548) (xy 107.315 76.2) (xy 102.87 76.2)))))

